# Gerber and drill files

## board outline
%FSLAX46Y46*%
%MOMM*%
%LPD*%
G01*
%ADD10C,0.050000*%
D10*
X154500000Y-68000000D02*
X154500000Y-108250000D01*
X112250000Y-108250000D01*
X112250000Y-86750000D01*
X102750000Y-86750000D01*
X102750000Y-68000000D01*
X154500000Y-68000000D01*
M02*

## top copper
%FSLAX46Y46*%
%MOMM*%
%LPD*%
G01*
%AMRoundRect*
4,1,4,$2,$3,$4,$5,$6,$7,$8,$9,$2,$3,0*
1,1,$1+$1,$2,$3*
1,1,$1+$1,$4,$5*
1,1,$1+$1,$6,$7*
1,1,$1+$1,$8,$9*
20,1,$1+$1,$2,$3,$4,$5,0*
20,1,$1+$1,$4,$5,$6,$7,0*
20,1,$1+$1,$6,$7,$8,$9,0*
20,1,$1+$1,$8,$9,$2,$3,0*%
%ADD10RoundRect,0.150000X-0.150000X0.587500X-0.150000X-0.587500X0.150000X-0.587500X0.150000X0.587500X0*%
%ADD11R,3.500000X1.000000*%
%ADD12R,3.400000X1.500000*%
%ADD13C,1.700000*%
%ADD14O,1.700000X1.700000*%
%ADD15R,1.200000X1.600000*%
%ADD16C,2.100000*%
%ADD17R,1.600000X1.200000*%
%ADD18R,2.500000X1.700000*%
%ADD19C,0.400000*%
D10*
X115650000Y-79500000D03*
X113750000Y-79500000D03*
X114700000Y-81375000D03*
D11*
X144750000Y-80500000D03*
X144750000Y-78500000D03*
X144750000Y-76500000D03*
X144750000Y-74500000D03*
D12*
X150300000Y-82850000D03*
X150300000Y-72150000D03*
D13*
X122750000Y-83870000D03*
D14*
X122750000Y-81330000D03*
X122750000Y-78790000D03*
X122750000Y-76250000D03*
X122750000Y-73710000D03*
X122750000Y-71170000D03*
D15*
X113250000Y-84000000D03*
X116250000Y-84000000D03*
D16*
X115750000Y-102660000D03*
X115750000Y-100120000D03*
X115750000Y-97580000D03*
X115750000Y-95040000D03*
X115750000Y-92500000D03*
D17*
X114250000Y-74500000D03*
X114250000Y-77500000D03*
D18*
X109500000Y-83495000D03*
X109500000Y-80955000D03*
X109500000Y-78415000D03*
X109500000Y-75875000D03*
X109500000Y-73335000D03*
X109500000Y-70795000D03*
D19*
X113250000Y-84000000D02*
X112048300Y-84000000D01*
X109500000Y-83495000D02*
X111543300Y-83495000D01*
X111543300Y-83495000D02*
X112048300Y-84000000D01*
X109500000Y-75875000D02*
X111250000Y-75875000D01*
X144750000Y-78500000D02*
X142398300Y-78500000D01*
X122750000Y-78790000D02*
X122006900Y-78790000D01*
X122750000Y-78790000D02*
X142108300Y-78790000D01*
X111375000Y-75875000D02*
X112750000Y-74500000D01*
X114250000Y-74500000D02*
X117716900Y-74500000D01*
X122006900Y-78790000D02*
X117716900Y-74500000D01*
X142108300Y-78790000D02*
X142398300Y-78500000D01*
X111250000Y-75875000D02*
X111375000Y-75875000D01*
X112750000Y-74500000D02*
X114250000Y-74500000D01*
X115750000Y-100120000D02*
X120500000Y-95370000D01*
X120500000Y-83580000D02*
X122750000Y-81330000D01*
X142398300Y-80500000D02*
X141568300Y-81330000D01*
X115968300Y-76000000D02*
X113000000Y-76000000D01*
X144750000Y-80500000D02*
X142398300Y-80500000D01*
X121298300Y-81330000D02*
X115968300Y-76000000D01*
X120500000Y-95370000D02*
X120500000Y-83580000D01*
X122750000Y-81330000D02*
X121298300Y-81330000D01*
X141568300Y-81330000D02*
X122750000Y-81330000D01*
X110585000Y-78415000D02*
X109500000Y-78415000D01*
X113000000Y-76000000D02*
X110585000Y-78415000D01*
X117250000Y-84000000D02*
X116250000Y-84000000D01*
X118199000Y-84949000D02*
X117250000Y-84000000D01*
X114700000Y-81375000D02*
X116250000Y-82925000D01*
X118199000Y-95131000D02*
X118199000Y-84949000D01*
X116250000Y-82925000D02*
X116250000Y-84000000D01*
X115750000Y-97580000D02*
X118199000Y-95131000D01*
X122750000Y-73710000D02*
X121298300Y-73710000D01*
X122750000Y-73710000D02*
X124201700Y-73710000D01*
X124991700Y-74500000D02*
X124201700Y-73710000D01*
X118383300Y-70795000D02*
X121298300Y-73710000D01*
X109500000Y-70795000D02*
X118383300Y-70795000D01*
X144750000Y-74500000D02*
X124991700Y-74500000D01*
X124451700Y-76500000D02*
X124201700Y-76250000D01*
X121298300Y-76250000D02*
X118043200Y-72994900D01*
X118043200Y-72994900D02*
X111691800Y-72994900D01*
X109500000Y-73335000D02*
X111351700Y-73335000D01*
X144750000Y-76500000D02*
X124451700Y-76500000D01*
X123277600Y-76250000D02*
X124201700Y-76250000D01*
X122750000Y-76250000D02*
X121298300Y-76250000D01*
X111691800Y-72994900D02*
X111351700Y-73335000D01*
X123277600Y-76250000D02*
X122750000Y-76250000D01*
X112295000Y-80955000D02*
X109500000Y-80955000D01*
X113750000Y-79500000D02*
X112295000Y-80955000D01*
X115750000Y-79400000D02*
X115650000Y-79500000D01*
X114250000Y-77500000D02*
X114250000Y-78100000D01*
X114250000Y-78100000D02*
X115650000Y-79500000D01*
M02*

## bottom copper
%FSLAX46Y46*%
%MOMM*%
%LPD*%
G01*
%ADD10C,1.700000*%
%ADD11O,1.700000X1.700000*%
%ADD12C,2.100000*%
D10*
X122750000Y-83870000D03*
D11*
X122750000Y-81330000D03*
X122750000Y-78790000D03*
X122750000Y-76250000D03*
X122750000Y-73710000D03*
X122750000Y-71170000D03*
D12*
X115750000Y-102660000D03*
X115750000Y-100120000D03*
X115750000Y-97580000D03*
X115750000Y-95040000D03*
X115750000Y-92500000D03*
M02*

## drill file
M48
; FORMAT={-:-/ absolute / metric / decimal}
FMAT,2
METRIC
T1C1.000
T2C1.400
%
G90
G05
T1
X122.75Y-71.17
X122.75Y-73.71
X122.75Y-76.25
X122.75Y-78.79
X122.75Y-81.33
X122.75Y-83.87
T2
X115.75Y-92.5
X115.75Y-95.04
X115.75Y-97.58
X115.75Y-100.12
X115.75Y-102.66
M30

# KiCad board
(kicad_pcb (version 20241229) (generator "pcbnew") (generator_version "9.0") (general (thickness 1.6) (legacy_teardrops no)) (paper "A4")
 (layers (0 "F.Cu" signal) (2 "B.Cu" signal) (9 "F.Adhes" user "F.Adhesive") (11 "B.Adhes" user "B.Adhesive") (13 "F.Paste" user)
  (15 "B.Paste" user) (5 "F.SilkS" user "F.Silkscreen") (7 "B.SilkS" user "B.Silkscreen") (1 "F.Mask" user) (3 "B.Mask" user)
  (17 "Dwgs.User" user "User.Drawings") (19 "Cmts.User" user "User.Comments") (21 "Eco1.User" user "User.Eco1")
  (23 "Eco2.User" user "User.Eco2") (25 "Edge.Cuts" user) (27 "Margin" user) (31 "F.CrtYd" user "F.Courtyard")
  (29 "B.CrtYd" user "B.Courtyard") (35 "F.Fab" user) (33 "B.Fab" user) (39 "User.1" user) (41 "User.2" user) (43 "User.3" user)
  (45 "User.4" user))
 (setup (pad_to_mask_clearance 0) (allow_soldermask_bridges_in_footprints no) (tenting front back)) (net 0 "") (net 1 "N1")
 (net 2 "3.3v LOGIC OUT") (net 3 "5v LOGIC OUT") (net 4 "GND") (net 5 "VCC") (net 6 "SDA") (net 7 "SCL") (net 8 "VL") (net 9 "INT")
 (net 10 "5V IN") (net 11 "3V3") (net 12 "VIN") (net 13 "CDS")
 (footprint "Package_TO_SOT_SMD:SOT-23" (layer "F.Cu") (at 114.7 80.4375 -90)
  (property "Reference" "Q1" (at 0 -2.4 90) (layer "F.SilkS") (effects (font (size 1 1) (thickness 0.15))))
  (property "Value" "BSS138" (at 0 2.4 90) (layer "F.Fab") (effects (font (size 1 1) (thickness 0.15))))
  (pad "1" smd roundrect (at -0.9375 -0.95 270) (size 1.475 0.6) (layers "F.Cu" "F.Mask" "F.Paste") (roundrect_rratio 0.25) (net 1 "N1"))
  (pad "2" smd roundrect (at -0.9375 0.95 270) (size 1.475 0.6) (layers "F.Cu" "F.Mask" "F.Paste") (roundrect_rratio 0.25)
   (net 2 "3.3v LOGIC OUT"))
  (pad "3" smd roundrect (at 0.9375 0 270) (size 1.475 0.6) (layers "F.Cu" "F.Mask" "F.Paste") (roundrect_rratio 0.25)
   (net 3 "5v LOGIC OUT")))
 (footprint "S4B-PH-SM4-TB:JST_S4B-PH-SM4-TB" (layer "F.Cu") (at 147.5 77.5 90)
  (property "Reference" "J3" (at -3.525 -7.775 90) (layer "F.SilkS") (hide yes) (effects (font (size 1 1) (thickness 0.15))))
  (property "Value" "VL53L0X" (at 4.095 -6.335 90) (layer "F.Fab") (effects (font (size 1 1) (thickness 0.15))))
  (pad "1" smd rect (at -3 -2.75 90) (size 1 3.5) (layers "F.Cu" "F.Mask" "F.Paste") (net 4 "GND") (solder_mask_margin 0.102))
  (pad "2" smd rect (at -1 -2.75 90) (size 1 3.5) (layers "F.Cu" "F.Mask" "F.Paste") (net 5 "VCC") (solder_mask_margin 0.102))
  (pad "3" smd rect (at 1 -2.75 90) (size 1 3.5) (layers "F.Cu" "F.Mask" "F.Paste") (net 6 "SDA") (solder_mask_margin 0.102))
  (pad "4" smd rect (at 3 -2.75 90) (size 1 3.5) (layers "F.Cu" "F.Mask" "F.Paste") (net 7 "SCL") (solder_mask_margin 0.102))
  (pad "SH1" smd rect (at -5.35 2.8 90) (size 1.5 3.4) (layers "F.Cu" "F.Mask" "F.Paste") (solder_mask_margin 0.102))
  (pad "SH2" smd rect (at 5.35 2.8 90) (size 1.5 3.4) (layers "F.Cu" "F.Mask" "F.Paste") (solder_mask_margin 0.102)))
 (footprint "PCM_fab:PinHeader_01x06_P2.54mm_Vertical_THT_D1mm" (layer "F.Cu") (at 122.75 83.87 180)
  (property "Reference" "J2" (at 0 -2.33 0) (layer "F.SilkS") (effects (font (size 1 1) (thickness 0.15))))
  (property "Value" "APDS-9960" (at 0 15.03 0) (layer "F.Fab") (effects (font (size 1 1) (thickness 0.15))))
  (pad "1" thru_hole circle (at 0 0 180) (size 1.7 1.7) (drill 1) (layers "*.Cu" "*.Mask") (remove_unused_layers no) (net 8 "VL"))
  (pad "2" thru_hole oval (at 0 2.54 180) (size 1.7 1.7) (drill 1) (layers "*.Cu" "*.Mask") (remove_unused_layers no) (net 4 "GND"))
  (pad "3" thru_hole oval (at 0 5.08 180) (size 1.7 1.7) (drill 1) (layers "*.Cu" "*.Mask") (remove_unused_layers no) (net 5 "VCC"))
  (pad "4" thru_hole oval (at 0 7.62 180) (size 1.7 1.7) (drill 1) (layers "*.Cu" "*.Mask") (remove_unused_layers no) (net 6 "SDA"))
  (pad "5" thru_hole oval (at 0 10.16 180) (size 1.7 1.7) (drill 1) (layers "*.Cu" "*.Mask") (remove_unused_layers no) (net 7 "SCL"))
  (pad "6" thru_hole oval (at 0 12.7 180) (size 1.7 1.7) (drill 1) (layers "*.Cu" "*.Mask") (remove_unused_layers no) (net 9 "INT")))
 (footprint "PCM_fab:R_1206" (layer "F.Cu") (at 114.75 84)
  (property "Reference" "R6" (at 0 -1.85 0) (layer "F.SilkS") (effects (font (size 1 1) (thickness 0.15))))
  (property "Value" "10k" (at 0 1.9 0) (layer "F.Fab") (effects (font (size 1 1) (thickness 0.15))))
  (pad "1" smd rect (at -1.5 0) (size 1.2 1.6) (layers "F.Cu" "F.Mask" "F.Paste") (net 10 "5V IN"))
  (pad "2" smd rect (at 1.5 0) (size 1.2 1.6) (layers "F.Cu" "F.Mask" "F.Paste") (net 3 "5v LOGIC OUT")))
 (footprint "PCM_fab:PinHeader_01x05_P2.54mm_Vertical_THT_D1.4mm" (layer "F.Cu") (at 115.75 102.66 180)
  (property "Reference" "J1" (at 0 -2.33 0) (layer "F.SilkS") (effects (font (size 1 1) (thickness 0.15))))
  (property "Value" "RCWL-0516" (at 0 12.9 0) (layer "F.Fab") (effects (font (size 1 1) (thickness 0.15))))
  (pad "1" thru_hole circle (at 0 0 180) (size 2.1 2.1) (drill 1.4) (layers "*.Cu" "*.Mask") (remove_unused_layers no) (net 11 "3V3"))
  (pad "2" thru_hole circle (at 0 2.54 180) (size 2.1 2.1) (drill 1.4) (layers "*.Cu" "*.Mask") (remove_unused_layers no) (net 4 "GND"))
  (pad "3" thru_hole circle (at 0 5.08 180) (size 2.1 2.1) (drill 1.4) (layers "*.Cu" "*.Mask") (remove_unused_layers no)
   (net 3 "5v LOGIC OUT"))
  (pad "4" thru_hole circle (at 0 7.62 180) (size 2.1 2.1) (drill 1.4) (layers "*.Cu" "*.Mask") (remove_unused_layers no) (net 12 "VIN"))
  (pad "5" thru_hole circle (at 0 10.16 180) (size 2.1 2.1) (drill 1.4) (layers "*.Cu" "*.Mask") (remove_unused_layers no) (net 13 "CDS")))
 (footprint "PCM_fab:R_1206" (layer "F.Cu") (at 114.25 76 -90)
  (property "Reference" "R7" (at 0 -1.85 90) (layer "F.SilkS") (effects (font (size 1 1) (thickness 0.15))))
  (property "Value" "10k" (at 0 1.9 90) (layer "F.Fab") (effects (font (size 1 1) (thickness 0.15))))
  (pad "1" smd rect (at -1.5 0 270) (size 1.2 1.6) (layers "F.Cu" "F.Mask" "F.Paste") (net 5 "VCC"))
  (pad "2" smd rect (at 1.5 0 270) (size 1.2 1.6) (layers "F.Cu" "F.Mask" "F.Paste") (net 1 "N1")))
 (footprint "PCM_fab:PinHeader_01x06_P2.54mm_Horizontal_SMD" (layer "F.Cu") (at 109.5 83.495 180)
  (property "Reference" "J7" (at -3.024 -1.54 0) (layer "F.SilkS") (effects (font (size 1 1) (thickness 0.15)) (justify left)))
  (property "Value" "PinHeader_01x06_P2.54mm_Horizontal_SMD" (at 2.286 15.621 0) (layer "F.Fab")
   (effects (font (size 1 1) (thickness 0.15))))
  (pad "1" smd rect (at 0 0 180) (size 2.5 1.7) (layers "F.Cu" "F.Mask" "F.Paste") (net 10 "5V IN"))
  (pad "2" smd rect (at 0 2.54 180) (size 2.5 1.7) (layers "F.Cu" "F.Mask" "F.Paste") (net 2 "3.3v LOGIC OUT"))
  (pad "3" smd rect (at 0 5.08 180) (size 2.5 1.7) (layers "F.Cu" "F.Mask" "F.Paste") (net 4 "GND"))
  (pad "4" smd rect (at 0 7.62 180) (size 2.5 1.7) (layers "F.Cu" "F.Mask" "F.Paste") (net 5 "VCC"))
  (pad "5" smd rect (at 0 10.16 180) (size 2.5 1.7) (layers "F.Cu" "F.Mask" "F.Paste") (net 6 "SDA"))
  (pad "6" smd rect (at 0 12.7 180) (size 2.5 1.7) (layers "F.Cu" "F.Mask" "F.Paste") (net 7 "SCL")))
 (gr_poly
  (pts (xy 154.5 68) (xy 154.5 108.25) (xy 112.25 108.25) (xy 112.25 86.75) (xy 102.75 86.75) (xy 102.75 68))
  (stroke (width 0.05) (type solid)) (fill no) (layer "Edge.Cuts"))
 (segment (start 113.25 84) (end 112.0483 84) (width 0.4) (layer "F.Cu") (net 10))
 (segment (start 109.5 83.495) (end 111.5433 83.495) (width 0.4) (layer "F.Cu") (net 10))
 (segment (start 111.5433 83.495) (end 112.0483 84) (width 0.4) (layer "F.Cu") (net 10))
 (segment (start 109.5 75.875) (end 111.25 75.875) (width 0.4) (layer "F.Cu") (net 5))
 (segment (start 144.75 78.5) (end 142.3983 78.5) (width 0.4) (layer "F.Cu") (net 5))
 (segment (start 122.75 78.79) (end 122.0069 78.79) (width 0.4) (layer "F.Cu") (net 5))
 (segment (start 122.75 78.79) (end 142.1083 78.79) (width 0.4) (layer "F.Cu") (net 5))
 (segment (start 111.375 75.875) (end 112.75 74.5) (width 0.4) (layer "F.Cu") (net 5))
 (segment (start 114.25 74.5) (end 117.7169 74.5) (width 0.4) (layer "F.Cu") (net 5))
 (segment (start 122.0069 78.79) (end 117.7169 74.5) (width 0.4) (layer "F.Cu") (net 5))
 (segment (start 142.1083 78.79) (end 142.3983 78.5) (width 0.4) (layer "F.Cu") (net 5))
 (segment (start 111.25 75.875) (end 111.375 75.875) (width 0.4) (layer "F.Cu") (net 5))
 (segment (start 112.75 74.5) (end 114.25 74.5) (width 0.4) (layer "F.Cu") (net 5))
 (segment (start 115.75 100.12) (end 120.5 95.37) (width 0.4) (layer "F.Cu") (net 4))
 (segment (start 120.5 83.58) (end 122.75 81.33) (width 0.4) (layer "F.Cu") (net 4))
 (segment (start 142.3983 80.5) (end 141.5683 81.33) (width 0.4) (layer "F.Cu") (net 4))
 (segment (start 115.9683 76) (end 113 76) (width 0.4) (layer "F.Cu") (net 4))
 (segment (start 144.75 80.5) (end 142.3983 80.5) (width 0.4) (layer "F.Cu") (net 4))
 (segment (start 121.2983 81.33) (end 115.9683 76) (width 0.4) (layer "F.Cu") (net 4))
 (segment (start 120.5 95.37) (end 120.5 83.58) (width 0.4) (layer "F.Cu") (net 4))
 (segment (start 122.75 81.33) (end 121.2983 81.33) (width 0.4) (layer "F.Cu") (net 4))
 (segment (start 141.5683 81.33) (end 122.75 81.33) (width 0.4) (layer "F.Cu") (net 4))
 (segment (start 110.585 78.415) (end 109.5 78.415) (width 0.4) (layer "F.Cu") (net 4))
 (segment (start 113 76) (end 110.585 78.415) (width 0.4) (layer "F.Cu") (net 4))
 (segment (start 117.25 84) (end 116.25 84) (width 0.4) (layer "F.Cu") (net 3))
 (segment (start 118.199 84.949) (end 117.25 84) (width 0.4) (layer "F.Cu") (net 3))
 (segment (start 114.7 81.375) (end 116.25 82.925) (width 0.4) (layer "F.Cu") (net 3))
 (segment (start 118.199 95.131) (end 118.199 84.949) (width 0.4) (layer "F.Cu") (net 3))
 (segment (start 116.25 82.925) (end 116.25 84) (width 0.4) (layer "F.Cu") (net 3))
 (segment (start 115.75 97.58) (end 118.199 95.131) (width 0.4) (layer "F.Cu") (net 3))
 (segment (start 122.75 73.71) (end 121.2983 73.71) (width 0.4) (layer "F.Cu") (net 7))
 (segment (start 122.75 73.71) (end 124.2017 73.71) (width 0.4) (layer "F.Cu") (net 7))
 (segment (start 124.9917 74.5) (end 124.2017 73.71) (width 0.4) (layer "F.Cu") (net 7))
 (segment (start 118.3833 70.795) (end 121.2983 73.71) (width 0.4) (layer "F.Cu") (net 7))
 (segment (start 109.5 70.795) (end 118.3833 70.795) (width 0.4) (layer "F.Cu") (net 7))
 (segment (start 144.75 74.5) (end 124.9917 74.5) (width 0.4) (layer "F.Cu") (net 7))
 (segment (start 124.4517 76.5) (end 124.2017 76.25) (width 0.4) (layer "F.Cu") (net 6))
 (segment (start 121.2983 76.25) (end 118.0432 72.9949) (width 0.4) (layer "F.Cu") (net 6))
 (segment (start 118.0432 72.9949) (end 111.6918 72.9949) (width 0.4) (layer "F.Cu") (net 6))
 (segment (start 109.5 73.335) (end 111.3517 73.335) (width 0.4) (layer "F.Cu") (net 6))
 (segment (start 144.75 76.5) (end 124.4517 76.5) (width 0.4) (layer "F.Cu") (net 6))
 (segment (start 123.2776 76.25) (end 124.2017 76.25) (width 0.4) (layer "F.Cu") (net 6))
 (segment (start 122.75 76.25) (end 121.2983 76.25) (width 0.4) (layer "F.Cu") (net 6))
 (segment (start 111.6918 72.9949) (end 111.3517 73.335) (width 0.4) (layer "F.Cu") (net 6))
 (segment (start 123.2776 76.25) (end 122.75 76.25) (width 0.4) (layer "F.Cu") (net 6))
 (segment (start 112.295 80.955) (end 109.5 80.955) (width 0.4) (layer "F.Cu") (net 2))
 (segment (start 113.75 79.5) (end 112.295 80.955) (width 0.4) (layer "F.Cu") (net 2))
 (segment (start 115.75 79.4) (end 115.65 79.5) (width 0.4) (layer "F.Cu") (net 1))
 (segment (start 114.25 77.5) (end 114.25 78.1) (width 0.4) (layer "F.Cu") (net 1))
 (segment (start 114.25 78.1) (end 115.65 79.5) (width 0.4) (layer "F.Cu") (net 1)))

